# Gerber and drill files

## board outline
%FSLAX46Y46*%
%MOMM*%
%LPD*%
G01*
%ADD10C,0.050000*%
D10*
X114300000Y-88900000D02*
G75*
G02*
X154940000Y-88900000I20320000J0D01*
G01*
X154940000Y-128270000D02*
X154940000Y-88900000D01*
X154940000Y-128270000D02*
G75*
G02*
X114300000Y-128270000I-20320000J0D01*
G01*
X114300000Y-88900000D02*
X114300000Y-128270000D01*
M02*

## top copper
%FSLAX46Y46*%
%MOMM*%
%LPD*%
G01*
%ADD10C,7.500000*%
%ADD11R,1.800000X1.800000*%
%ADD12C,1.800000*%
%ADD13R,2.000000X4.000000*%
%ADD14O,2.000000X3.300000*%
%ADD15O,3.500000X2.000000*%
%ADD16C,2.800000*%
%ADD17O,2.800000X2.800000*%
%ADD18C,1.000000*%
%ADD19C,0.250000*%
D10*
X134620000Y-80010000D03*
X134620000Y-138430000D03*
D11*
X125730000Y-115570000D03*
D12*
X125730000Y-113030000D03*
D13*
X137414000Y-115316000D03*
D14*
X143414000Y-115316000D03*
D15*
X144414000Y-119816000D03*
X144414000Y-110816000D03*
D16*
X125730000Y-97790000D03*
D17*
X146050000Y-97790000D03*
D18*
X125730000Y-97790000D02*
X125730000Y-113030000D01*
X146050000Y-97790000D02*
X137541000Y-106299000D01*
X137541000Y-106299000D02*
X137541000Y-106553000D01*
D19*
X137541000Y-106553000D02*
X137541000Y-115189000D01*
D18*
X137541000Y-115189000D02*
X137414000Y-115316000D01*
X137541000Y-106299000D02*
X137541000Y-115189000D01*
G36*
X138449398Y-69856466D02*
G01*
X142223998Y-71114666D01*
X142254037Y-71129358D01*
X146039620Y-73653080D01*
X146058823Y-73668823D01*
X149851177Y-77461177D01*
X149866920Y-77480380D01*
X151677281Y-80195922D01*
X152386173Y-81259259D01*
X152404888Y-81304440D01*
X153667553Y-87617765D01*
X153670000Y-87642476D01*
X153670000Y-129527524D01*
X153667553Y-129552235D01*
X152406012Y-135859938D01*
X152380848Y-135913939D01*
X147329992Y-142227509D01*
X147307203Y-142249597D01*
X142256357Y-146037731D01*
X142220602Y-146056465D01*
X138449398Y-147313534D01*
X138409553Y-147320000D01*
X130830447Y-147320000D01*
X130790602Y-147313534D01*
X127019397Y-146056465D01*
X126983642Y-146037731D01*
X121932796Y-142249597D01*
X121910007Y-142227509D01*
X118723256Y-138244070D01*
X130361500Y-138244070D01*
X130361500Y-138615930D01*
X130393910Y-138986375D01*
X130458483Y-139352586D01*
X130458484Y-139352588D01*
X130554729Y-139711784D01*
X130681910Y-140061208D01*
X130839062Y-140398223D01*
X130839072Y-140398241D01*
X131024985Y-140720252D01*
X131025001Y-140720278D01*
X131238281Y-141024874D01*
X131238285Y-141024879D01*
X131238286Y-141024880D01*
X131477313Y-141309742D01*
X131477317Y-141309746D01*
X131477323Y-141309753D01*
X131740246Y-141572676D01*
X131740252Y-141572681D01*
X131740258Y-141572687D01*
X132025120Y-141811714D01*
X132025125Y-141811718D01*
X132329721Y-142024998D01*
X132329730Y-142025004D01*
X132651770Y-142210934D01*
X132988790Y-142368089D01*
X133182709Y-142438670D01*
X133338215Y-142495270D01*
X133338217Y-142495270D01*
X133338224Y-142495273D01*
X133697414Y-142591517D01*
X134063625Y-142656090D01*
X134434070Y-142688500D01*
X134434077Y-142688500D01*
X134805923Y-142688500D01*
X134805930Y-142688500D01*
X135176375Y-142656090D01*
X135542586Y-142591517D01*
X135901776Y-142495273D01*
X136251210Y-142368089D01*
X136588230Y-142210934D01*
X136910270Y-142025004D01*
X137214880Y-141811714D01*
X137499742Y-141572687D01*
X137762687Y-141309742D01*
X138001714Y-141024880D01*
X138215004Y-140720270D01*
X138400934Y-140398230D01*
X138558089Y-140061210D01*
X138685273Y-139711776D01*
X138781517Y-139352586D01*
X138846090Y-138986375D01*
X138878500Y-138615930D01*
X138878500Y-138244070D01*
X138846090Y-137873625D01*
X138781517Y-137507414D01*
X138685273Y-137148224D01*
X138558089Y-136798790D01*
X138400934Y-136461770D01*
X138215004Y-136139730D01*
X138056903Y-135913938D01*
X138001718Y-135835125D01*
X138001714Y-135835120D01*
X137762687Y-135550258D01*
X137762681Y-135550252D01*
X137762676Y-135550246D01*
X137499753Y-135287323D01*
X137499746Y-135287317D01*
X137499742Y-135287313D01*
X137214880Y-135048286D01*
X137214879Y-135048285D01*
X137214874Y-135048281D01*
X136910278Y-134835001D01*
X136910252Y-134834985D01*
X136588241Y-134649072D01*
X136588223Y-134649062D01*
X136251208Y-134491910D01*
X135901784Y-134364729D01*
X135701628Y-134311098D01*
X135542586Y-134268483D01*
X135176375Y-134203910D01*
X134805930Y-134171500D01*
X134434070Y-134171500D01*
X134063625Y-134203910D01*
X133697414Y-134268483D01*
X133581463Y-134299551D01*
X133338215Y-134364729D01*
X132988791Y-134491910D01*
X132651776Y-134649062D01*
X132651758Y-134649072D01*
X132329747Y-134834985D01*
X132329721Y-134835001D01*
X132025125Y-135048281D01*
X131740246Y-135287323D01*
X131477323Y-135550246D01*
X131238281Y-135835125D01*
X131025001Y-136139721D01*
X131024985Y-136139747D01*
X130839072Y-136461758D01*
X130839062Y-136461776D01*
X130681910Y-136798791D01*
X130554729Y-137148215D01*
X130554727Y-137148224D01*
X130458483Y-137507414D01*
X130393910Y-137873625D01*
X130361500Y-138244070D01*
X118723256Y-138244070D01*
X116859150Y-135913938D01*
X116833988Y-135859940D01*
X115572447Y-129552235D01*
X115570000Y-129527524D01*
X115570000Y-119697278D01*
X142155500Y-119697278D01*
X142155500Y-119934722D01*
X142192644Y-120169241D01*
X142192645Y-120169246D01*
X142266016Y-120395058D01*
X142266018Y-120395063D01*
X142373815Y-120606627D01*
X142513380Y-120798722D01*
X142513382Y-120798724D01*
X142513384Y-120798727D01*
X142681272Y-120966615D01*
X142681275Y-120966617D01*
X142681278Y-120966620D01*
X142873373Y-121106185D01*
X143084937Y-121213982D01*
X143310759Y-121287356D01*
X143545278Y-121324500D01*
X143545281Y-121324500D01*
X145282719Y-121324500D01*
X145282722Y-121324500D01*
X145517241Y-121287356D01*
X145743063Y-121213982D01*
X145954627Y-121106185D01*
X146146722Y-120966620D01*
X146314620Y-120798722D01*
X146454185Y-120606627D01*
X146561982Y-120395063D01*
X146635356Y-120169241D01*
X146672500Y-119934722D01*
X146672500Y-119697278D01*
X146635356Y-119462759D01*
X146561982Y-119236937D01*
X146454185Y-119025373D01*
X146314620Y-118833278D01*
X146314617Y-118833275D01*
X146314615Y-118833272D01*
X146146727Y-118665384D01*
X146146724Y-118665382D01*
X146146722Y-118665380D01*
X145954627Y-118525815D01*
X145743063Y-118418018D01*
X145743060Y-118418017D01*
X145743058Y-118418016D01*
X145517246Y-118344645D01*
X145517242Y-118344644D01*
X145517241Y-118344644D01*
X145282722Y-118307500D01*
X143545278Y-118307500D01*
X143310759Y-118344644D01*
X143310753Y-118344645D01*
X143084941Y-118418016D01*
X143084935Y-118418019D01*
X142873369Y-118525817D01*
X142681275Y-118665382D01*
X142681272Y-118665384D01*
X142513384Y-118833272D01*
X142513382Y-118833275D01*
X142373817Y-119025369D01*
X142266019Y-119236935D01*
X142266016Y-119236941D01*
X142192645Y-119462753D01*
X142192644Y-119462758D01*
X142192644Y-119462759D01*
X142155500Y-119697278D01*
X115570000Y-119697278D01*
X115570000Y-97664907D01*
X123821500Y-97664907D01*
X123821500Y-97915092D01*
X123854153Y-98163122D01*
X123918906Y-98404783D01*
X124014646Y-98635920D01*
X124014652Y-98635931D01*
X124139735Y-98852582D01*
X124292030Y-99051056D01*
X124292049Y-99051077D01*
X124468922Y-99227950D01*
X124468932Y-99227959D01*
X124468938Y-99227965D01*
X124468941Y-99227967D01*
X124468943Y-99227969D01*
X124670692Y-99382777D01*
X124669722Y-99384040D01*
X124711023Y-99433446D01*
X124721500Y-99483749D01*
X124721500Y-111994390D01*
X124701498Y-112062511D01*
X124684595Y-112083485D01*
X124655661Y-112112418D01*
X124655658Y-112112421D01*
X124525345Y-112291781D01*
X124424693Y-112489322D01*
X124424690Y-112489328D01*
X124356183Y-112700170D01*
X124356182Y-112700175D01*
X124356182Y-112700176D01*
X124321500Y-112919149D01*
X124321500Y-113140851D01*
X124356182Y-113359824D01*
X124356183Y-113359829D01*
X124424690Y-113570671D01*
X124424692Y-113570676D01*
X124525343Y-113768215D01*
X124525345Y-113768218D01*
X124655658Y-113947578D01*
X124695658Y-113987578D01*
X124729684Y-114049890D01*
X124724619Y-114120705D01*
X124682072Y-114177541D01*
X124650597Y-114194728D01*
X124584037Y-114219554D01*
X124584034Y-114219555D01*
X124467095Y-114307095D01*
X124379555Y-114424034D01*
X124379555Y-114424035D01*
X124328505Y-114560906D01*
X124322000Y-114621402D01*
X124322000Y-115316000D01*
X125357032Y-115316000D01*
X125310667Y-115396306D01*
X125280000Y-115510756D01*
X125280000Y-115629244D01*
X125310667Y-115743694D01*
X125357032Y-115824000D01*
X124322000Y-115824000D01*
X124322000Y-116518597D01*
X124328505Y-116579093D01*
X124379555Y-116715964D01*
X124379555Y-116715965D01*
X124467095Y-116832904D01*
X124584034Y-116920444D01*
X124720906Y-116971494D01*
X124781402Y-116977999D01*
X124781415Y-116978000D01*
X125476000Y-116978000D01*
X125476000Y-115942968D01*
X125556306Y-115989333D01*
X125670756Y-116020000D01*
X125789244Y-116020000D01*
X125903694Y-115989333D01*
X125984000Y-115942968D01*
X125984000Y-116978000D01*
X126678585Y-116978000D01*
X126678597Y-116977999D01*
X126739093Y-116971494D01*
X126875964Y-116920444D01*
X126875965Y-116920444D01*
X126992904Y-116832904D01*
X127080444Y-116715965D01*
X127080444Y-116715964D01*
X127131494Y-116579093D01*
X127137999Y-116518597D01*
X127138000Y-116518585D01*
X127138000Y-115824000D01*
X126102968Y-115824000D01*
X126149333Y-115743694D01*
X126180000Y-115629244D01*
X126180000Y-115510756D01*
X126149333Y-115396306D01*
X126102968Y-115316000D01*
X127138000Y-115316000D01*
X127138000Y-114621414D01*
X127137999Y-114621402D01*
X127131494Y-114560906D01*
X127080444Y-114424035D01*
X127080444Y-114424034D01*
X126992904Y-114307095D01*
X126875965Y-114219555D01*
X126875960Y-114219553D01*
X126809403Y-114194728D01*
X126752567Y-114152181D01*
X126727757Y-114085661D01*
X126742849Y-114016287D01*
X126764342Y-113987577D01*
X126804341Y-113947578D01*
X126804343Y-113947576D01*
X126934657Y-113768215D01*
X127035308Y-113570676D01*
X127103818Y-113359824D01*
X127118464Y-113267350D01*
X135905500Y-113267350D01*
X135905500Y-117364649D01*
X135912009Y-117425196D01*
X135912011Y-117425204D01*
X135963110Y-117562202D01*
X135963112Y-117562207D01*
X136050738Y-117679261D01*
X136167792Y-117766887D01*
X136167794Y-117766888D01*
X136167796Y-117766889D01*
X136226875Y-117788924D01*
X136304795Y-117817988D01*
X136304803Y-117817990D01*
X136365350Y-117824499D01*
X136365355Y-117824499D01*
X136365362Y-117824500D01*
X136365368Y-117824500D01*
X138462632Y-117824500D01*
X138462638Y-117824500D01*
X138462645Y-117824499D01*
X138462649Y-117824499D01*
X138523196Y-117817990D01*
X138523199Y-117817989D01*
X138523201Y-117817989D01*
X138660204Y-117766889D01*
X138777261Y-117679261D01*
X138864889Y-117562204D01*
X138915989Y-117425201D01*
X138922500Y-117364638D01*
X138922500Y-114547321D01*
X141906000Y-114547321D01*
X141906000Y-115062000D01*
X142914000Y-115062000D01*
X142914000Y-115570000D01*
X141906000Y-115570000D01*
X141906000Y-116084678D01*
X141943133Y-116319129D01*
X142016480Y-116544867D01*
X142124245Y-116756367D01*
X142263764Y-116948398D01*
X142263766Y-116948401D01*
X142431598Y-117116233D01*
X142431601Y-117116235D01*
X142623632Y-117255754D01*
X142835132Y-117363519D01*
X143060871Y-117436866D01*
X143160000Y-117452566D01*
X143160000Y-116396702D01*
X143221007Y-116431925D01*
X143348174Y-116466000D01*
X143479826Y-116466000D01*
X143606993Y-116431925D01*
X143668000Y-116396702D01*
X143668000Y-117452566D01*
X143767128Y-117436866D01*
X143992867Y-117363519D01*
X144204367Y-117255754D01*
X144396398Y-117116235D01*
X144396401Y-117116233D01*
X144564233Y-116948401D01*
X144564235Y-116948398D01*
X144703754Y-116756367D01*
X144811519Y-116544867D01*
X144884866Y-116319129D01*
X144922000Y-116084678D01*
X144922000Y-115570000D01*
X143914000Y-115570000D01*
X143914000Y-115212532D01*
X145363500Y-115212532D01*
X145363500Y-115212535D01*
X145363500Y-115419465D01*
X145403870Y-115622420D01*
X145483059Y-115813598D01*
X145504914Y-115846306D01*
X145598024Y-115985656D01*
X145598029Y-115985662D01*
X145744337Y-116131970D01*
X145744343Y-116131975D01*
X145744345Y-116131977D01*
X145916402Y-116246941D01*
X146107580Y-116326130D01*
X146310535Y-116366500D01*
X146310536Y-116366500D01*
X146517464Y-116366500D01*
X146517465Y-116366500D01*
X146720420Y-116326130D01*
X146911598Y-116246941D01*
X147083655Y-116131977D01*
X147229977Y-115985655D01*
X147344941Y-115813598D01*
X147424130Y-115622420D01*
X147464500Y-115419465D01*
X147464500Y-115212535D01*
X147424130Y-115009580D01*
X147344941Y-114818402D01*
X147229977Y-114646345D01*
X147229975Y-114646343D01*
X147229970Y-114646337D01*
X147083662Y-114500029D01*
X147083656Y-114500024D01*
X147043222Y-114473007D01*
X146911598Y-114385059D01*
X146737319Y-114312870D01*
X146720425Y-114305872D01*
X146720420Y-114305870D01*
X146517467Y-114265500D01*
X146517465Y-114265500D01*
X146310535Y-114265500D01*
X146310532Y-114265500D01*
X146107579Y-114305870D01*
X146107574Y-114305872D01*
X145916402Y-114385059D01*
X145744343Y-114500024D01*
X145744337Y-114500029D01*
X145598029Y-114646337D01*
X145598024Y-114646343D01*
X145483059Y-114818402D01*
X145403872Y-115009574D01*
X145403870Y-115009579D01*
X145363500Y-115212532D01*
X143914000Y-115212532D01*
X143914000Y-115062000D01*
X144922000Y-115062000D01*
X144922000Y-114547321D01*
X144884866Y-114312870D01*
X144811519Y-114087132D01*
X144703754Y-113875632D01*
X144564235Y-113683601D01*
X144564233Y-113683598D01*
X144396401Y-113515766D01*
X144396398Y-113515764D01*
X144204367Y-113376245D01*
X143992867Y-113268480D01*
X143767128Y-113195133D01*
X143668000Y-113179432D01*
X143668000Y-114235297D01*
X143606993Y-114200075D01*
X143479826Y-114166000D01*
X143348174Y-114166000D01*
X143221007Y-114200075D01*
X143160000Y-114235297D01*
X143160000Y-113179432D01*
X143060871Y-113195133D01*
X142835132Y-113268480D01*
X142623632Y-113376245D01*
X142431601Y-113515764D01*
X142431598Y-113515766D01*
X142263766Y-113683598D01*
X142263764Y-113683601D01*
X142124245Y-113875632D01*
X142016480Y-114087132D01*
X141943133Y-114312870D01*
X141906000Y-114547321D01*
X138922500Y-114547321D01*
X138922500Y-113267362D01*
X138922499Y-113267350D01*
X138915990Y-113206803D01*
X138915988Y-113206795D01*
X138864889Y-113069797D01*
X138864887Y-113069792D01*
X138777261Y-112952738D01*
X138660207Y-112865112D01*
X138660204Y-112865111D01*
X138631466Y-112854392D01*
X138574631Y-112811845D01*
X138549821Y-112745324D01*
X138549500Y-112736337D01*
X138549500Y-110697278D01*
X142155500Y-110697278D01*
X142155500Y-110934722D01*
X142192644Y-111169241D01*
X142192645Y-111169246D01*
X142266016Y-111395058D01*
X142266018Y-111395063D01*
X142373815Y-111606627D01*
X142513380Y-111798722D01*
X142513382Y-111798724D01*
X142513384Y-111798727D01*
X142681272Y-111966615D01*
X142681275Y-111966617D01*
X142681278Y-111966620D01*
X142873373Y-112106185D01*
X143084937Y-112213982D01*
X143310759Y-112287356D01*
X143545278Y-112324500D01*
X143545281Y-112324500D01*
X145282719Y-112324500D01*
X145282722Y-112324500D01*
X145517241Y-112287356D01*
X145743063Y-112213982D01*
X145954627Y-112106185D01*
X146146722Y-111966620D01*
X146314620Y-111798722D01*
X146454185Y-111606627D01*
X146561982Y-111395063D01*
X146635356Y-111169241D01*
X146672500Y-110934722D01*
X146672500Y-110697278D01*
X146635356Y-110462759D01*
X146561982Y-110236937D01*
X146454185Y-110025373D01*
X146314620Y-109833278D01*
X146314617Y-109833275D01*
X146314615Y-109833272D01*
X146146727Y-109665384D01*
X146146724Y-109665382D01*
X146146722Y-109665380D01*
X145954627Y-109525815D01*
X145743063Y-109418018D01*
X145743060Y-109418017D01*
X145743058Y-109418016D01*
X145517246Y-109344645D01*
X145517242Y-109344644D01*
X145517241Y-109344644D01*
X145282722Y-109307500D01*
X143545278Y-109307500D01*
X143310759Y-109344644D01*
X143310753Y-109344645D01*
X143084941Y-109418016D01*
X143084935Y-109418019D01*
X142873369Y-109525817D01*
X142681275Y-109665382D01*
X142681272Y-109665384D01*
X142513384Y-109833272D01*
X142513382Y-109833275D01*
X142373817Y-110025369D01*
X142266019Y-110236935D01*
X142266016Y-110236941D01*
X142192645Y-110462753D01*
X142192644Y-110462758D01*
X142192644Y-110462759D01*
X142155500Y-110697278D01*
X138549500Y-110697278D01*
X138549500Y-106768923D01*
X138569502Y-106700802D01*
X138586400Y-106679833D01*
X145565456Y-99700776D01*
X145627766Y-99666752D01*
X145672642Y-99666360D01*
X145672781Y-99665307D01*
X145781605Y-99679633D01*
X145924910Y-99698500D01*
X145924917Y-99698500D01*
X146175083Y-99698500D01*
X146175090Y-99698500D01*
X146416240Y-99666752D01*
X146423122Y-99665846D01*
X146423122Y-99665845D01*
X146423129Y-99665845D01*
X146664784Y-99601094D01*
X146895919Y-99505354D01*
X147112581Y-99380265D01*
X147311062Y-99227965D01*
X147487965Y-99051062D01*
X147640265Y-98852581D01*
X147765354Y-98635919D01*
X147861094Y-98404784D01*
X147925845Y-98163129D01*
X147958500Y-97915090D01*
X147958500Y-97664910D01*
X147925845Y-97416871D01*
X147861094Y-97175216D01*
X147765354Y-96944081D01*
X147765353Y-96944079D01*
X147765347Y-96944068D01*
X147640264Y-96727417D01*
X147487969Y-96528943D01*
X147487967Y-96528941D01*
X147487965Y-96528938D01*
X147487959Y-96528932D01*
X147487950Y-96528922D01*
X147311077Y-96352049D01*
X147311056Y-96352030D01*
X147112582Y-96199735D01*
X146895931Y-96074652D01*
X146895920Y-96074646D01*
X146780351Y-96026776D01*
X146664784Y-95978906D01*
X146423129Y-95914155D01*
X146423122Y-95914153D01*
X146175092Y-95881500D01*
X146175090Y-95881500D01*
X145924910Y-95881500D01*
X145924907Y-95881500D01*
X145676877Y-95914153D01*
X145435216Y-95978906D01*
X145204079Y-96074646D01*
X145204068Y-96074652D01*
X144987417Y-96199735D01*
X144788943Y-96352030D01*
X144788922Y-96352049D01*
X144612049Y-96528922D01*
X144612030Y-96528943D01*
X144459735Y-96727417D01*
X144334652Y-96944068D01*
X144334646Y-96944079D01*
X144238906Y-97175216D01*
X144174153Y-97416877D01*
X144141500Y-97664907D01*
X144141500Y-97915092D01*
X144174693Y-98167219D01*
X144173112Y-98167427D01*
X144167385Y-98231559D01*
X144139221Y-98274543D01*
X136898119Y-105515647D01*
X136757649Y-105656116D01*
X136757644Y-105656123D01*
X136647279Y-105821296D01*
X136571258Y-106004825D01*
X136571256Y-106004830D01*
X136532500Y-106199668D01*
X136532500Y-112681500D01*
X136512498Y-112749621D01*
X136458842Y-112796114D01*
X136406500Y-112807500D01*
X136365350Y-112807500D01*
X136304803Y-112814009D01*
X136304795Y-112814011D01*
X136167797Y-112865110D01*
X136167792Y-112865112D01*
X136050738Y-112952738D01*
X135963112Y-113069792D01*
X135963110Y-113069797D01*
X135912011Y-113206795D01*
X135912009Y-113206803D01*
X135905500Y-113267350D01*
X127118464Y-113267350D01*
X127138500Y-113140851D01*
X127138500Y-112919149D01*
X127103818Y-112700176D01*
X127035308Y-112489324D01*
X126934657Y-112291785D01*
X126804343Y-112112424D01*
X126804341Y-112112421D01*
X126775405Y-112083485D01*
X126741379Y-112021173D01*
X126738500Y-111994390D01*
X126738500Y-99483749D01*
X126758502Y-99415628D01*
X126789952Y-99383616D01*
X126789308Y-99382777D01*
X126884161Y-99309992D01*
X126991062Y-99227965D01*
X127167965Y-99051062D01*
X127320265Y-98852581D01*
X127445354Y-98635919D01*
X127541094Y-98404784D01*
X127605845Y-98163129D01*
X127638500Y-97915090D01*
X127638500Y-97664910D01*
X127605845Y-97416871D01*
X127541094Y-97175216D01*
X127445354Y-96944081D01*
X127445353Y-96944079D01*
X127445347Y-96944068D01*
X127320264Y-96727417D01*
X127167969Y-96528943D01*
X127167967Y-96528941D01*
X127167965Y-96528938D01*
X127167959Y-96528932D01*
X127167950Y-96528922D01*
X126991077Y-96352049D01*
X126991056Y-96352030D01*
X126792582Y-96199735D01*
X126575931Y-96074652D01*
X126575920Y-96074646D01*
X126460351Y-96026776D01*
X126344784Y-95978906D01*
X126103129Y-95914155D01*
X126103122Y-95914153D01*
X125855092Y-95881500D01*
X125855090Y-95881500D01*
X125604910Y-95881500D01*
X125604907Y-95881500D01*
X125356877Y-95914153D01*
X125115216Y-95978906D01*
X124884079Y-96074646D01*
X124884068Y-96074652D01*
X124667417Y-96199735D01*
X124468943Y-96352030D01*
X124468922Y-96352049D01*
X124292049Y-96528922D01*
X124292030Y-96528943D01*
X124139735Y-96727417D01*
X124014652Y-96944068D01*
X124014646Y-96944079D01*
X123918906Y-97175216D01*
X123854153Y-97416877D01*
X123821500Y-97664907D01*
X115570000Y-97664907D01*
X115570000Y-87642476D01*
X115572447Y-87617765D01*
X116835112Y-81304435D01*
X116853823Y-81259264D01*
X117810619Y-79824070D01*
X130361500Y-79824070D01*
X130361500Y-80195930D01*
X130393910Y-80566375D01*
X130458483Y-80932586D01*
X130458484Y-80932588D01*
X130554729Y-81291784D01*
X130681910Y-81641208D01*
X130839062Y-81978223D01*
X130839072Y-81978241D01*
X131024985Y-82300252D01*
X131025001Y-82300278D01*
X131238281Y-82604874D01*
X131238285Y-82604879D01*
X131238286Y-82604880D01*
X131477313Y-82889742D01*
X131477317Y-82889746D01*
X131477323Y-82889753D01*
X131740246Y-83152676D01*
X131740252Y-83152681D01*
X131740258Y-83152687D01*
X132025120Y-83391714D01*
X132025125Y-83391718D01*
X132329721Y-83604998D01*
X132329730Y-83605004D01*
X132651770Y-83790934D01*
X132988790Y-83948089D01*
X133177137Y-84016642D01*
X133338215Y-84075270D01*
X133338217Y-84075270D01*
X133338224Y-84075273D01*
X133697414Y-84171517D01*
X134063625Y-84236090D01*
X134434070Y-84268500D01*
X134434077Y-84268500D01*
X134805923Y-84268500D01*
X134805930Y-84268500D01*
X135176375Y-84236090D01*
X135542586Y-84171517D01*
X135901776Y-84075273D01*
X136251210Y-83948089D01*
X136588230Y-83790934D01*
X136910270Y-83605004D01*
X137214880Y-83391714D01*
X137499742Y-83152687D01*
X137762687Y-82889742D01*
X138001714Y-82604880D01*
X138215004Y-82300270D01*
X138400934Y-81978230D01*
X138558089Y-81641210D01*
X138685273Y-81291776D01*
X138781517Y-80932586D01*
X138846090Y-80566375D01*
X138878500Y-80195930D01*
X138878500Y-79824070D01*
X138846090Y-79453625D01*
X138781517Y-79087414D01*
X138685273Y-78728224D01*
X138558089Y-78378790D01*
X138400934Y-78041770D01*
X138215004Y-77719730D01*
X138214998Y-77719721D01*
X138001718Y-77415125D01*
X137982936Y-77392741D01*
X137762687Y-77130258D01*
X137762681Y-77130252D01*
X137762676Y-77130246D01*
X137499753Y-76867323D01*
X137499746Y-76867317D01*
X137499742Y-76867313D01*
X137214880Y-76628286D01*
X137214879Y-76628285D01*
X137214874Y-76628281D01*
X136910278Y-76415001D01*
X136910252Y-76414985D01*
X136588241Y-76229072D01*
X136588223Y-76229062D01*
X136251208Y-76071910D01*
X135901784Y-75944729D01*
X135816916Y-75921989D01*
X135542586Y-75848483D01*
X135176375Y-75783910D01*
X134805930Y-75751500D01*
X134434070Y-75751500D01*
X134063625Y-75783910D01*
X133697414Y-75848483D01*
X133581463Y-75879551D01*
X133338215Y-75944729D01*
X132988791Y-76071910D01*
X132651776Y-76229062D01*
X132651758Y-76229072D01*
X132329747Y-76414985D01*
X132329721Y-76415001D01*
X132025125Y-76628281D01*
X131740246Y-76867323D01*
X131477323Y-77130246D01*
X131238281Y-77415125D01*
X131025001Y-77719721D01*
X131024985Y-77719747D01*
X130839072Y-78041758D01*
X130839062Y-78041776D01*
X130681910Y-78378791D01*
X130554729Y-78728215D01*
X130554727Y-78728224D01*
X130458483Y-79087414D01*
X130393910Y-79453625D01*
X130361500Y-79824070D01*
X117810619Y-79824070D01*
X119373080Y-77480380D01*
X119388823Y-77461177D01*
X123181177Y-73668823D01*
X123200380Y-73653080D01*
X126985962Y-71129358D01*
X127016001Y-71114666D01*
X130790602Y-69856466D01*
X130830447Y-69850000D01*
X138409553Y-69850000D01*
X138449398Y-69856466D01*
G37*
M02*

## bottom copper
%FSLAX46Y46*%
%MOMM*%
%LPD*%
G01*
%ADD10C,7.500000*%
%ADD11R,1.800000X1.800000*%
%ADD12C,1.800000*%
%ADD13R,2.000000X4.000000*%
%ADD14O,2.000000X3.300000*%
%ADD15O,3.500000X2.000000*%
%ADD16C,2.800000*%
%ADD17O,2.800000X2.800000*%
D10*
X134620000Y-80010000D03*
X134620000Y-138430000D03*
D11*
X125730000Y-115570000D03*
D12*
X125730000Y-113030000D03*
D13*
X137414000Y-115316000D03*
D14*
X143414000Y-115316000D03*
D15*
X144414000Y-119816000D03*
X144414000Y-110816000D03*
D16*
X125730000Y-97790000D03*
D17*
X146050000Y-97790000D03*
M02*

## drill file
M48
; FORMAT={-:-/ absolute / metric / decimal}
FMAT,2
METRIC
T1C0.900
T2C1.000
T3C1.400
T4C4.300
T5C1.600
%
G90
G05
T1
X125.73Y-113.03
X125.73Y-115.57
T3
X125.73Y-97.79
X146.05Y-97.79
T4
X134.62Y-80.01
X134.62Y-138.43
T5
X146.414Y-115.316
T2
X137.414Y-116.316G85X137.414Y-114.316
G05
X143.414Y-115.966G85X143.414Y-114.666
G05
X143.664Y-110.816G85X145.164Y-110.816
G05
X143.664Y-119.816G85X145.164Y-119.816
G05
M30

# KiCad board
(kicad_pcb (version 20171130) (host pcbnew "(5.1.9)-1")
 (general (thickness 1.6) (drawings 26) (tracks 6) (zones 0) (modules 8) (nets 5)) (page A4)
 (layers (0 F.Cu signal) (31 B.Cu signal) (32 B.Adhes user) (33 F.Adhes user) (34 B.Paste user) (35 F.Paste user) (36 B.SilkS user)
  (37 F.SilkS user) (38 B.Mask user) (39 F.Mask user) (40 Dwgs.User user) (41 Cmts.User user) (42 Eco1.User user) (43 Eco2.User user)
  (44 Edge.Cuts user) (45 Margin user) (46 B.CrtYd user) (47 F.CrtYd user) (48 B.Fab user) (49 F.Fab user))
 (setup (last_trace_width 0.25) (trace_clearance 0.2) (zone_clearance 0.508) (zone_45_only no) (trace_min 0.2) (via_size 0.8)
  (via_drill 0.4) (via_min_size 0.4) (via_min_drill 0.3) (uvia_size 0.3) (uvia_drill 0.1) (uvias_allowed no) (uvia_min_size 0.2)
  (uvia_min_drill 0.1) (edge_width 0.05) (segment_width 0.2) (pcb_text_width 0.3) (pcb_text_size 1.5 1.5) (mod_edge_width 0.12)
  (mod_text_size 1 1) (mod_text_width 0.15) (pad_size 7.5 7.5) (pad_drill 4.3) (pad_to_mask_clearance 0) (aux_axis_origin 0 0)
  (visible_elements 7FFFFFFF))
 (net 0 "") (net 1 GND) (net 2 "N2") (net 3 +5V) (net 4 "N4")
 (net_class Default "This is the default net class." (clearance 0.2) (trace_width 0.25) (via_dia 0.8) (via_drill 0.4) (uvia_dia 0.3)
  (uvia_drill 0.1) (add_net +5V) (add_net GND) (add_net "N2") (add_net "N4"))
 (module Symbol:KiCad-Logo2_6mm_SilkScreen (layer B.Cu) (at 141.986 126.619 180)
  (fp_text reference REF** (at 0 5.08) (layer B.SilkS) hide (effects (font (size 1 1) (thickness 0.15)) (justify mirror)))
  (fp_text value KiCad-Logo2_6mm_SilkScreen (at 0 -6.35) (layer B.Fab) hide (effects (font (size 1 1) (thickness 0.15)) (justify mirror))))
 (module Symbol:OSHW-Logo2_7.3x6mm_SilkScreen (layer F.Cu) (at 123.952 127)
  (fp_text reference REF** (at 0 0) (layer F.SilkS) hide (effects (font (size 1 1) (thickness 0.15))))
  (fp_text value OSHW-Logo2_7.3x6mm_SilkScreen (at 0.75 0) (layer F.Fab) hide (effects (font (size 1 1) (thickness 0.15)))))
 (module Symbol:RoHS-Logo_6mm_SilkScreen (layer B.Cu) (at 139.573 104.775 180)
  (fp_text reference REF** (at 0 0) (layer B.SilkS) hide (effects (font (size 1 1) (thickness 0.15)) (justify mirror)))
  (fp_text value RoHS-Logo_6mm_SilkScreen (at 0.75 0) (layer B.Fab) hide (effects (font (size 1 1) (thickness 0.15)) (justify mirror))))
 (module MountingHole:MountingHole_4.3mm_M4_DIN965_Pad (layer F.Cu) (at 134.62 80.01)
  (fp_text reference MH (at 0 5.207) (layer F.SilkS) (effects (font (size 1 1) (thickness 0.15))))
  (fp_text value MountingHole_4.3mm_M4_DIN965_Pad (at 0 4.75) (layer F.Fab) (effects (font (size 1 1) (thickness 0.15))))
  (pad 1 thru_hole circle (at 0 0) (size 7.5 7.5) (drill 4.3) (layers *.Cu *.Mask)))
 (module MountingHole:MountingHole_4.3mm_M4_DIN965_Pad (layer F.Cu) (at 134.62 138.43)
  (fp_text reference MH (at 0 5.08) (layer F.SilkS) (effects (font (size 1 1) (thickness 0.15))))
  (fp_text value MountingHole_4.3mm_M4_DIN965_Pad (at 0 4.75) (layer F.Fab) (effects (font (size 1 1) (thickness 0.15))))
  (pad 1 thru_hole circle (at 0 0) (size 7.5 7.5) (drill 4.3) (layers *.Cu *.Mask)))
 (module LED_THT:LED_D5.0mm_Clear (layer F.Cu) (at 125.73 115.57 90)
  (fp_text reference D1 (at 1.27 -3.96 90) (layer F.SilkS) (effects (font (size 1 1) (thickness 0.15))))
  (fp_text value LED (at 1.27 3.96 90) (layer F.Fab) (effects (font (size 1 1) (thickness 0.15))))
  (pad 1 thru_hole rect (at 0 0 90) (size 1.8 1.8) (drill 0.9) (layers *.Cu *.Mask) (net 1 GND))
  (pad 2 thru_hole circle (at 2.54 0 90) (size 1.8 1.8) (drill 0.9) (layers *.Cu *.Mask) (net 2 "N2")))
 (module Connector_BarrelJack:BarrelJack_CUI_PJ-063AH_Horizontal (layer F.Cu) (at 137.414 115.316 90)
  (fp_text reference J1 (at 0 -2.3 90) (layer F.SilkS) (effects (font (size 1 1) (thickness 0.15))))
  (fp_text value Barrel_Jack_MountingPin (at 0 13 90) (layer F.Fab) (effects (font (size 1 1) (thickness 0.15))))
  (pad 1 thru_hole rect (at 0 0 90) (size 4 2) (drill oval 3 1) (layers *.Cu *.Mask) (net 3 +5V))
  (pad 2 thru_hole oval (at 0 6 90) (size 3.3 2) (drill oval 2.3 1) (layers *.Cu *.Mask) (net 1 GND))
  (pad MP thru_hole oval (at -4.5 7 90) (size 2 3.5) (drill oval 1 2.5) (layers *.Cu *.Mask) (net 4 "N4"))
  (pad MP thru_hole oval (at 4.5 7 90) (size 2 3.5) (drill oval 1 2.5) (layers *.Cu *.Mask) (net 4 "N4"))
  (pad "" np_thru_hole circle (at 0 9 90) (size 1.6 1.6) (drill 1.6) (layers *.Cu *.Mask)))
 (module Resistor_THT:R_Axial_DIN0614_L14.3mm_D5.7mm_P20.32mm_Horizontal (layer F.Cu) (at 125.73 97.79)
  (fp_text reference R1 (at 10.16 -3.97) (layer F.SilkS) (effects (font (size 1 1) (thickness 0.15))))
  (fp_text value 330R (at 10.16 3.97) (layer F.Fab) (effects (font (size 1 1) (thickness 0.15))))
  (pad 1 thru_hole circle (at 0 0) (size 2.8 2.8) (drill 1.4) (layers *.Cu *.Mask) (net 2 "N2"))
  (pad 2 thru_hole oval (at 20.32 0) (size 2.8 2.8) (drill 1.4) (layers *.Cu *.Mask) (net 3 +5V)))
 (gr_arc (start 134.62 88.9) (end 154.94 88.9) (angle -180) (layer Edge.Cuts) (width 0.05))
 (gr_line (start 154.94 128.27) (end 154.94 88.9) (layer Edge.Cuts) (width 0.05))
 (gr_arc (start 134.62 128.27) (end 114.3 128.27) (angle -180) (layer Edge.Cuts) (width 0.05))
 (gr_line (start 114.3 88.9) (end 114.3 128.27) (layer Edge.Cuts) (width 0.05))
 (segment (start 125.73 97.79) (end 125.73 113.03) (width 1) (layer F.Cu) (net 2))
 (segment (start 146.05 97.79) (end 137.541 106.299) (width 1) (layer F.Cu) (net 3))
 (segment (start 137.541 106.299) (end 137.541 106.553) (width 1) (layer F.Cu) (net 3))
 (segment (start 137.541 106.553) (end 137.541 115.189) (width 0.25) (layer F.Cu) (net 3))
 (segment (start 137.541 115.189) (end 137.414 115.316) (width 1) (layer F.Cu) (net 3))
 (segment (start 137.541 106.299) (end 137.541 115.189) (width 1) (layer F.Cu) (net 3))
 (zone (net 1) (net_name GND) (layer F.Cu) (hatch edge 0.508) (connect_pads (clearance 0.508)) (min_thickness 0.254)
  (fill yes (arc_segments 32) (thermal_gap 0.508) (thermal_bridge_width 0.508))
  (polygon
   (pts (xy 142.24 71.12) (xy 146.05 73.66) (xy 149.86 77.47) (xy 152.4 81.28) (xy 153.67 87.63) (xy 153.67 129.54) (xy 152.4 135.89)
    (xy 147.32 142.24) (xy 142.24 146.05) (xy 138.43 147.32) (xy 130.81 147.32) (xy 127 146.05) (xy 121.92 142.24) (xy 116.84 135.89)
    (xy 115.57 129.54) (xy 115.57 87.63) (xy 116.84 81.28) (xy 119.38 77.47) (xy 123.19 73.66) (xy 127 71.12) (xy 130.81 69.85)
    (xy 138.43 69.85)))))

